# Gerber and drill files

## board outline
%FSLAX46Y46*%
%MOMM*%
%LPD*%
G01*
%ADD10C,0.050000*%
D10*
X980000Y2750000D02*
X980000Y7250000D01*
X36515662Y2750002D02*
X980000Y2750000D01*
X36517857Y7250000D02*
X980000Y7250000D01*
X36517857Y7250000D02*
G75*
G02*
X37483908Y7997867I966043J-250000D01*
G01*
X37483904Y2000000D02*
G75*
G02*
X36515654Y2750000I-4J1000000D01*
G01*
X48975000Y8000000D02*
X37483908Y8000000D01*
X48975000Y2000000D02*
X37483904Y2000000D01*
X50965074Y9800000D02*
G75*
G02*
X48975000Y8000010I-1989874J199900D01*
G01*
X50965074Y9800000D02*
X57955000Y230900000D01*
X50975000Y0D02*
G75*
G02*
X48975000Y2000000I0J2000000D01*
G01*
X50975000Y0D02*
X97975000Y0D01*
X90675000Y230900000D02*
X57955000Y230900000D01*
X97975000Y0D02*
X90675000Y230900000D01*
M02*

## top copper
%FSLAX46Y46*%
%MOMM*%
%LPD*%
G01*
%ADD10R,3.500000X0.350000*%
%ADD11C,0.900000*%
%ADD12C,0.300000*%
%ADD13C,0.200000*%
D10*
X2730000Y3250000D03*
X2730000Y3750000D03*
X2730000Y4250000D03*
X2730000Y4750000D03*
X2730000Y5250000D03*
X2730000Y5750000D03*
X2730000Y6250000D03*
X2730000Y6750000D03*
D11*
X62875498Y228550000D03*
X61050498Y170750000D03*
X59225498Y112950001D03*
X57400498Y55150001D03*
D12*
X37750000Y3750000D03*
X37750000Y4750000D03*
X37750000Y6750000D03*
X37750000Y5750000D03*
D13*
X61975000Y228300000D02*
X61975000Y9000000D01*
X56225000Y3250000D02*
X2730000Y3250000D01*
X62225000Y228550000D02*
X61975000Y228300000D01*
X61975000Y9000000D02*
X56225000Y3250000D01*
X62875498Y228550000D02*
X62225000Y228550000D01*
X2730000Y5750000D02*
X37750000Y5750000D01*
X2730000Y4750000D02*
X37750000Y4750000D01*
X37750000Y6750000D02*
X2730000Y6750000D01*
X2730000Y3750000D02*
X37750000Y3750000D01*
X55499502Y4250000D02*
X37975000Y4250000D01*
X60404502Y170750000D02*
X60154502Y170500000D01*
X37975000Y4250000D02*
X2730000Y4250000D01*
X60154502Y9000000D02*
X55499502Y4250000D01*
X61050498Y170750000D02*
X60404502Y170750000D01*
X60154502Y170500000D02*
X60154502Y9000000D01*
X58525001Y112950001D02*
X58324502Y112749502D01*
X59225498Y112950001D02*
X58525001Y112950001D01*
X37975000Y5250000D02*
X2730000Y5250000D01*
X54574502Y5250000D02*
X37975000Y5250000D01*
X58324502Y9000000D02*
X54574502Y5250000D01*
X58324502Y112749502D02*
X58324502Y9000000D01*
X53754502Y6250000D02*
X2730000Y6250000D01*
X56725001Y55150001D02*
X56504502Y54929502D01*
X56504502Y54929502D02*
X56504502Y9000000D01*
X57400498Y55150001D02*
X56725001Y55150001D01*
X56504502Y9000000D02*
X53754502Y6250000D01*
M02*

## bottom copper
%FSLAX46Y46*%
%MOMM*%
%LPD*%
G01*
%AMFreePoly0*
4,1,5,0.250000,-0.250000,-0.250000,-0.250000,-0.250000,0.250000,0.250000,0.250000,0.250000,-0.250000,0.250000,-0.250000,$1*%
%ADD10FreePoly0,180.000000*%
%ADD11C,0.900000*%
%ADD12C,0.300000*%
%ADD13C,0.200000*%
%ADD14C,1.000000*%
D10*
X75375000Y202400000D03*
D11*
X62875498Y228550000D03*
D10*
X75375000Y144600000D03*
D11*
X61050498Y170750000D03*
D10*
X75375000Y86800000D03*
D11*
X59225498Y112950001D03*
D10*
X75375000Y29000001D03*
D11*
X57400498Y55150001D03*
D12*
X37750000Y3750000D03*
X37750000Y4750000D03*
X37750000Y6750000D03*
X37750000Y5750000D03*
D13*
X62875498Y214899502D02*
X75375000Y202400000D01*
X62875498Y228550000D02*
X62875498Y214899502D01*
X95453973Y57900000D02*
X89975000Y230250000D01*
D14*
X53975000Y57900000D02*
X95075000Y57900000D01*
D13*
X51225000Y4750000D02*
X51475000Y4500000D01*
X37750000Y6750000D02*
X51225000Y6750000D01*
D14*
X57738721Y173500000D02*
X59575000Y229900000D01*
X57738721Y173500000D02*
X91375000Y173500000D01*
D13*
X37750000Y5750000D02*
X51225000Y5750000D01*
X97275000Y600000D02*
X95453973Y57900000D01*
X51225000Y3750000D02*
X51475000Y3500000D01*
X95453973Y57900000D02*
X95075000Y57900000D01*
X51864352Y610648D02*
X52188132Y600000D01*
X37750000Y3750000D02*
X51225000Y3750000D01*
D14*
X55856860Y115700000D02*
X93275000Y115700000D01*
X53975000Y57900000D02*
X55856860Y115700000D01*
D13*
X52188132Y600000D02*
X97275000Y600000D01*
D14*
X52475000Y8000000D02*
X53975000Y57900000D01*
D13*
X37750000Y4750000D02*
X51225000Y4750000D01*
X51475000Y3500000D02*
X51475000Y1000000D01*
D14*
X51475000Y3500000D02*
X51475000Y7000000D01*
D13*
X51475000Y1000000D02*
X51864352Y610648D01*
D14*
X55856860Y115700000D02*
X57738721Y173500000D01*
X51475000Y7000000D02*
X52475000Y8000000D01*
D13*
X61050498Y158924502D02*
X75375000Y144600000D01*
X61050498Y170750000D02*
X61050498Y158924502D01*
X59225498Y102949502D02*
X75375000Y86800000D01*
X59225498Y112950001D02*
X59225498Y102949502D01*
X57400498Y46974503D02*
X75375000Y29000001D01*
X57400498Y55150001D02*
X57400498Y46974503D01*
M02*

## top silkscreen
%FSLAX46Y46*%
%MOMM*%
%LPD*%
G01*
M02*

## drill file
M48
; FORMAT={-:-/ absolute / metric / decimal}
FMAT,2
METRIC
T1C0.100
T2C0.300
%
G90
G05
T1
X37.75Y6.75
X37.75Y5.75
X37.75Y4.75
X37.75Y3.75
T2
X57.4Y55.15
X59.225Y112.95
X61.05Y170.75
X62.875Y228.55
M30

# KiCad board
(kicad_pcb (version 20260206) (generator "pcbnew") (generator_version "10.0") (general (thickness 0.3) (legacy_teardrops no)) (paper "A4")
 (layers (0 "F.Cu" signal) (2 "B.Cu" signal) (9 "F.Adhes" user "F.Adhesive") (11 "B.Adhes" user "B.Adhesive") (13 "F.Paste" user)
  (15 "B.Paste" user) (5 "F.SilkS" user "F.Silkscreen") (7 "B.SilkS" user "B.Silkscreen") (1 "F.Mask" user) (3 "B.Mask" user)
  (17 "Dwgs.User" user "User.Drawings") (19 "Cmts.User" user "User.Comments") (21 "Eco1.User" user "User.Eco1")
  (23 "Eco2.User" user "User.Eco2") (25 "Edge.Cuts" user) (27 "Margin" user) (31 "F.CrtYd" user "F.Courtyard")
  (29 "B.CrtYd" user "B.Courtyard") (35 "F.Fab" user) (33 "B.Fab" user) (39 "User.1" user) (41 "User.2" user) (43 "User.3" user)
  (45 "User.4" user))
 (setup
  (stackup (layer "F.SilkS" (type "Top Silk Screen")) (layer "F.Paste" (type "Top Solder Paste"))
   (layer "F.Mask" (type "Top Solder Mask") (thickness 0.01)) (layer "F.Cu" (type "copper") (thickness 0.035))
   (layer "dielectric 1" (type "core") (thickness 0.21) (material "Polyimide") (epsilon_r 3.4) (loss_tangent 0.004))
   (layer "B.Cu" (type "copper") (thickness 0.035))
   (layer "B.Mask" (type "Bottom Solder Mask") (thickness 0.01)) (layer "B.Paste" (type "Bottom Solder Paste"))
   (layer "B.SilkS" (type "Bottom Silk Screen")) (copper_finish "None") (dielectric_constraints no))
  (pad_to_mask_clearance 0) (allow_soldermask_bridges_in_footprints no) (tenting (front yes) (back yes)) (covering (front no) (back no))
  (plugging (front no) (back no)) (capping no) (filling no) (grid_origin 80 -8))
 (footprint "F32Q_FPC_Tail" (layer "F.Cu") (at 0.98 -5 90)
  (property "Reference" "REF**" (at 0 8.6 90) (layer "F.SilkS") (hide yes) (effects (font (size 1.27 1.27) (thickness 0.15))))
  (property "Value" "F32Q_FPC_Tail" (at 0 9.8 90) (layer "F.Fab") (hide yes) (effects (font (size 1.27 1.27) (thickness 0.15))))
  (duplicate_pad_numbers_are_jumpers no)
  (pad "1" smd rect (at -1.75 1.75 90) (size 0.35 3.5) (layers "F.Cu" "F.Mask") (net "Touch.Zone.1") (thermal_bridge_angle 45))
  (pad "2" smd rect (at -1.25 1.75 90) (size 0.35 3.5) (layers "F.Cu" "F.Mask") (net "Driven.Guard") (thermal_bridge_angle 45))
  (pad "3" smd rect (at -0.75 1.75 90) (size 0.35 3.5) (layers "F.Cu" "F.Mask") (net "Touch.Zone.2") (thermal_bridge_angle 45))
  (pad "4" smd rect (at -0.25 1.75 90) (size 0.35 3.5) (layers "F.Cu" "F.Mask") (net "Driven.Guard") (thermal_bridge_angle 45))
  (pad "5" smd rect (at 0.25 1.75 90) (size 0.35 3.5) (layers "F.Cu" "F.Mask") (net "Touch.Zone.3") (thermal_bridge_angle 45))
  (pad "6" smd rect (at 0.75 1.75 90) (size 0.35 3.5) (layers "F.Cu" "F.Mask") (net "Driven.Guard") (thermal_bridge_angle 45))
  (pad "7" smd rect (at 1.25 1.75 90) (size 0.35 3.5) (layers "F.Cu" "F.Mask") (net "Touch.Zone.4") (thermal_bridge_angle 45))
  (pad "8" smd rect (at 1.75 1.75 90) (size 0.35 3.5) (layers "F.Cu" "F.Mask") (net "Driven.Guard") (thermal_bridge_angle 45)))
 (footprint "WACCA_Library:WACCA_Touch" (layer "B.Cu") (at 75.375 -202.4 180)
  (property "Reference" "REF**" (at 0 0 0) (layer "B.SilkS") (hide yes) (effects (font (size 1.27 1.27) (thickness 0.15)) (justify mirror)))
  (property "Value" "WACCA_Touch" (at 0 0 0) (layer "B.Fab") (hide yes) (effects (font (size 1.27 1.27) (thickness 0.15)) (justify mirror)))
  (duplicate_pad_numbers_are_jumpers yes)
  (pad "1" smd custom (at 0 0 180) (size 0.5 0.5) (layers "B.Cu" "B.Mask") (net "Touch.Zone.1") (thermal_bridge_angle 45)
   (options (clearance outline) (anchor rect)) (primitives))
  (pad "1" thru_hole circle (at 12.499502 26.15 180) (size 0.9 0.9) (drill 0.3) (layers "*.Cu" "*.Mask") (remove_unused_layers no)
   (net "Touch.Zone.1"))
  (pad "2" smd custom (at 0 -57.8 180) (size 0.5 0.5) (layers "B.Cu" "B.Mask") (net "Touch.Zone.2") (thermal_bridge_angle 45)
   (options (clearance outline) (anchor rect)) (primitives))
  (pad "2" thru_hole circle (at 14.324502 -31.65 180) (size 0.9 0.9) (drill 0.3) (layers "*.Cu" "*.Mask") (remove_unused_layers no)
   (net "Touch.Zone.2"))
  (pad "3" smd custom (at 0 -115.6 180) (size 0.5 0.5) (layers "B.Cu" "B.Mask") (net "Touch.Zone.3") (thermal_bridge_angle 45)
   (options (clearance outline) (anchor rect)) (primitives))
  (pad "3" thru_hole circle (at 16.149502 -89.449999 180) (size 0.9 0.9) (drill 0.3) (layers "*.Cu" "*.Mask") (remove_unused_layers no)
   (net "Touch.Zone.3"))
  (pad "4" smd custom (at 0 -173.399999 180) (size 0.5 0.5) (layers "B.Cu" "B.Mask") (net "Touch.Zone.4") (thermal_bridge_angle 45)
   (options (clearance outline) (anchor rect)) (primitives))
  (pad "4" thru_hole circle (at 17.974502 -147.249999 180) (size 0.9 0.9) (drill 0.3) (layers "*.Cu" "*.Mask") (remove_unused_layers no)
   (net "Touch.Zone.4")))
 (gr_line (start 0.98 -2.75) (end 0.98 -7.25) (stroke (width 0.05) (type default)) (layer "Edge.Cuts"))
 (gr_line (start 36.515662 -2.750002) (end 0.98 -2.75) (stroke (width 0.05) (type default)) (layer "Edge.Cuts"))
 (gr_line (start 36.517857 -7.25) (end 0.98 -7.25) (stroke (width 0.05) (type default)) (layer "Edge.Cuts"))
 (gr_arc (start 36.517857 -7.25) (mid 36.873054 -7.789054) (end 37.483908 -7.997867) (stroke (width 0.05) (type default))
  (layer "Edge.Cuts"))
 (gr_arc (start 37.483904 -2) (mid 36.871533 -2.209432) (end 36.515662 -2.750002) (stroke (width 0.05) (type default)) (layer "Edge.Cuts"))
 (gr_line (start 48.975 -8) (end 37.483908 -8) (stroke (width 0.05) (type default)) (layer "Edge.Cuts"))
 (gr_line (start 48.975 -2) (end 37.483904 -2) (stroke (width 0.05) (type default)) (layer "Edge.Cuts"))
 (gr_arc (start 50.965074 -9.8) (mid 50.316711 -8.51669) (end 48.975 -8) (stroke (width 0.05) (type default)) (layer "Edge.Cuts"))
 (gr_line (start 50.965074 -9.8) (end 57.955 -230.9) (stroke (width 0.05) (type default)) (layer "Edge.Cuts"))
 (gr_arc (start 50.975 0) (mid 49.560786 -0.585786) (end 48.975 -2) (stroke (width 0.05) (type default)) (layer "Edge.Cuts"))
 (gr_line (start 50.975 0) (end 97.975 0) (stroke (width 0.05) (type default)) (layer "Edge.Cuts"))
 (gr_line (start 90.675 -230.9) (end 57.955 -230.9) (stroke (width 0.05) (type default)) (layer "Edge.Cuts"))
 (gr_line (start 97.975 0) (end 90.675 -230.9) (stroke (width 0.05) (type default)) (layer "Edge.Cuts"))
 (segment (start 61.975 -228.3) (end 61.975 -9) (width 0.2) (layer "F.Cu") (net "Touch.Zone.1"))
 (segment (start 56.225 -3.25) (end 2.73 -3.25) (width 0.2) (layer "F.Cu") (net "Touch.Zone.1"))
 (segment (start 62.225 -228.55) (end 61.975 -228.3) (width 0.2) (layer "F.Cu") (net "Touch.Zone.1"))
 (segment (start 61.975 -9) (end 56.225 -3.25) (width 0.2) (layer "F.Cu") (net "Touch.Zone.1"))
 (segment (start 62.875498 -228.55) (end 62.225 -228.55) (width 0.2) (layer "F.Cu") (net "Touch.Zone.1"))
 (segment (start 62.875498 -214.899502) (end 75.375 -202.4) (width 0.2) (layer "B.Cu") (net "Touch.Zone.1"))
 (segment (start 62.875498 -228.55) (end 62.875498 -214.899502) (width 0.2) (layer "B.Cu") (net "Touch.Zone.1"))
 (segment (start 2.73 -5.75) (end 37.75 -5.75) (width 0.2) (layer "F.Cu") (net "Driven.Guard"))
 (segment (start 2.73 -4.75) (end 37.75 -4.75) (width 0.2) (layer "F.Cu") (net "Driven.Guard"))
 (segment (start 37.75 -6.75) (end 2.73 -6.75) (width 0.2) (layer "F.Cu") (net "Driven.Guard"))
 (segment (start 2.73 -3.75) (end 37.75 -3.75) (width 0.2) (layer "F.Cu") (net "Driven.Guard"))
 (via micro (at 37.75 -3.75) (size 0.3) (drill 0.1) (layers "F.Cu" "B.Cu") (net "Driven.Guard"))
 (via micro (at 37.75 -4.75) (size 0.3) (drill 0.1) (layers "F.Cu" "B.Cu") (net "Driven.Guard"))
 (via micro (at 37.75 -6.75) (size 0.3) (drill 0.1) (layers "F.Cu" "B.Cu") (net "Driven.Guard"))
 (via micro (at 37.75 -5.75) (size 0.3) (drill 0.1) (layers "F.Cu" "B.Cu") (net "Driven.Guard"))
 (segment (start 95.453973 -57.9) (end 89.975 -230.25) (width 0.2) (layer "B.Cu") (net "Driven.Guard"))
 (segment (start 53.975 -57.9) (end 95.075 -57.9) (width 1) (layer "B.Cu") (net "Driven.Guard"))
 (segment (start 51.225 -4.75) (end 51.475 -4.5) (width 0.2) (layer "B.Cu") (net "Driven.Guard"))
 (segment (start 37.75 -6.75) (end 51.225 -6.75) (width 0.2) (layer "B.Cu") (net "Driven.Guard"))
 (segment (start 57.738721 -173.5) (end 59.575 -229.9) (width 1) (layer "B.Cu") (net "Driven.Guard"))
 (segment (start 57.738721 -173.5) (end 91.375 -173.5) (width 1) (layer "B.Cu") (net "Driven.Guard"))
 (segment (start 37.75 -5.75) (end 51.225 -5.75) (width 0.2) (layer "B.Cu") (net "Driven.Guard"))
 (segment (start 97.275 -0.6) (end 95.453973 -57.9) (width 0.2) (layer "B.Cu") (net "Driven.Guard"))
 (segment (start 51.225 -3.75) (end 51.475 -3.5) (width 0.2) (layer "B.Cu") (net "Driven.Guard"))
 (segment (start 95.453973 -57.9) (end 95.075 -57.9) (width 0.2) (layer "B.Cu") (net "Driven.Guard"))
 (segment (start 51.864352 -0.610648) (end 52.188132 -0.6) (width 0.2) (layer "B.Cu") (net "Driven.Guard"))
 (segment (start 37.75 -3.75) (end 51.225 -3.75) (width 0.2) (layer "B.Cu") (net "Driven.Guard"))
 (segment (start 55.85686 -115.7) (end 93.275 -115.7) (width 1) (layer "B.Cu") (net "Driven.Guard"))
 (segment (start 53.975 -57.9) (end 55.85686 -115.7) (width 1) (layer "B.Cu") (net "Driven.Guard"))
 (segment (start 52.188132 -0.6) (end 97.275 -0.6) (width 0.2) (layer "B.Cu") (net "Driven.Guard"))
 (segment (start 52.475 -8) (end 53.975 -57.9) (width 1) (layer "B.Cu") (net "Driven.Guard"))
 (segment (start 37.75 -4.75) (end 51.225 -4.75) (width 0.2) (layer "B.Cu") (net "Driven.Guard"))
 (segment (start 51.475 -3.5) (end 51.475 -1) (width 0.2) (layer "B.Cu") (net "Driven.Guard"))
 (segment (start 51.475 -3.5) (end 51.475 -7) (width 1) (layer "B.Cu") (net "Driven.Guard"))
 (segment (start 51.475 -1) (end 51.864352 -0.610648) (width 0.2) (layer "B.Cu") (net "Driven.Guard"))
 (segment (start 55.85686 -115.7) (end 57.738721 -173.5) (width 1) (layer "B.Cu") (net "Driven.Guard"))
 (segment (start 51.475 -7) (end 52.475 -8) (width 1) (layer "B.Cu") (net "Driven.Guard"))
 (segment (start 55.499502 -4.25) (end 37.975 -4.25) (width 0.2) (layer "F.Cu") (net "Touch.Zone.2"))
 (segment (start 60.404502 -170.75) (end 60.154502 -170.5) (width 0.2) (layer "F.Cu") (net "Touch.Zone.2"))
 (segment (start 37.975 -4.25) (end 2.73 -4.25) (width 0.2) (layer "F.Cu") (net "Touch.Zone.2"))
 (segment (start 60.154502 -9) (end 55.499502 -4.25) (width 0.2) (layer "F.Cu") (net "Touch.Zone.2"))
 (segment (start 61.050498 -170.75) (end 60.404502 -170.75) (width 0.2) (layer "F.Cu") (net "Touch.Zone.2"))
 (segment (start 60.154502 -170.5) (end 60.154502 -9) (width 0.2) (layer "F.Cu") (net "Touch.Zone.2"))
 (segment (start 61.050498 -158.924502) (end 75.375 -144.6) (width 0.2) (layer "B.Cu") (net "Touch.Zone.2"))
 (segment (start 61.050498 -170.75) (end 61.050498 -158.924502) (width 0.2) (layer "B.Cu") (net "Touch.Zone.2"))
 (segment (start 58.525001 -112.950001) (end 58.324502 -112.749502) (width 0.2) (layer "F.Cu") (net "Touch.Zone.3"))
 (segment (start 59.225498 -112.950001) (end 58.525001 -112.950001) (width 0.2) (layer "F.Cu") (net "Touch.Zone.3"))
 (segment (start 37.975 -5.25) (end 2.73 -5.25) (width 0.2) (layer "F.Cu") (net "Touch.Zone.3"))
 (segment (start 54.574502 -5.25) (end 37.975 -5.25) (width 0.2) (layer "F.Cu") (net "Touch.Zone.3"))
 (segment (start 58.324502 -9) (end 54.574502 -5.25) (width 0.2) (layer "F.Cu") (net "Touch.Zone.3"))
 (segment (start 58.324502 -112.749502) (end 58.324502 -9) (width 0.2) (layer "F.Cu") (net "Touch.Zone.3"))
 (segment (start 59.225498 -102.949502) (end 75.375 -86.8) (width 0.2) (layer "B.Cu") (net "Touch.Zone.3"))
 (segment (start 59.225498 -112.950001) (end 59.225498 -102.949502) (width 0.2) (layer "B.Cu") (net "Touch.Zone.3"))
 (segment (start 53.754502 -6.25) (end 2.73 -6.25) (width 0.2) (layer "F.Cu") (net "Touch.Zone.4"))
 (segment (start 56.725001 -55.150001) (end 56.504502 -54.929502) (width 0.2) (layer "F.Cu") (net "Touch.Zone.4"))
 (segment (start 56.504502 -54.929502) (end 56.504502 -9) (width 0.2) (layer "F.Cu") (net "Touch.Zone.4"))
 (segment (start 57.400498 -55.150001) (end 56.725001 -55.150001) (width 0.2) (layer "F.Cu") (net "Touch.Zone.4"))
 (segment (start 56.504502 -9) (end 53.754502 -6.25) (width 0.2) (layer "F.Cu") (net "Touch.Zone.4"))
 (segment (start 57.400498 -46.974503) (end 75.375 -29.000001) (width 0.2) (layer "B.Cu") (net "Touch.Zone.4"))
 (segment (start 57.400498 -55.150001) (end 57.400498 -46.974503) (width 0.2) (layer "B.Cu") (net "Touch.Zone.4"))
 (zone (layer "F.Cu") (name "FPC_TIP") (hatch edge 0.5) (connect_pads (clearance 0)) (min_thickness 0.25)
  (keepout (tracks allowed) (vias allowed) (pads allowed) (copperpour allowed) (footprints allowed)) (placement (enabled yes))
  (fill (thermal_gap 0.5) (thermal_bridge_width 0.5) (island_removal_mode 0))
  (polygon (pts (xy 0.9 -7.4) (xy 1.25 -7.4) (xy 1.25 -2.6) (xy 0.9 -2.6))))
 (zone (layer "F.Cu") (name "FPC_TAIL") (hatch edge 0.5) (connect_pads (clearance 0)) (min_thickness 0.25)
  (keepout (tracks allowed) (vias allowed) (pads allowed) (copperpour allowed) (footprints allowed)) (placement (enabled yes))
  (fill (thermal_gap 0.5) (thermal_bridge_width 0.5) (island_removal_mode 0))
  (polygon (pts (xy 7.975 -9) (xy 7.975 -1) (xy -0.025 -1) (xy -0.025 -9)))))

